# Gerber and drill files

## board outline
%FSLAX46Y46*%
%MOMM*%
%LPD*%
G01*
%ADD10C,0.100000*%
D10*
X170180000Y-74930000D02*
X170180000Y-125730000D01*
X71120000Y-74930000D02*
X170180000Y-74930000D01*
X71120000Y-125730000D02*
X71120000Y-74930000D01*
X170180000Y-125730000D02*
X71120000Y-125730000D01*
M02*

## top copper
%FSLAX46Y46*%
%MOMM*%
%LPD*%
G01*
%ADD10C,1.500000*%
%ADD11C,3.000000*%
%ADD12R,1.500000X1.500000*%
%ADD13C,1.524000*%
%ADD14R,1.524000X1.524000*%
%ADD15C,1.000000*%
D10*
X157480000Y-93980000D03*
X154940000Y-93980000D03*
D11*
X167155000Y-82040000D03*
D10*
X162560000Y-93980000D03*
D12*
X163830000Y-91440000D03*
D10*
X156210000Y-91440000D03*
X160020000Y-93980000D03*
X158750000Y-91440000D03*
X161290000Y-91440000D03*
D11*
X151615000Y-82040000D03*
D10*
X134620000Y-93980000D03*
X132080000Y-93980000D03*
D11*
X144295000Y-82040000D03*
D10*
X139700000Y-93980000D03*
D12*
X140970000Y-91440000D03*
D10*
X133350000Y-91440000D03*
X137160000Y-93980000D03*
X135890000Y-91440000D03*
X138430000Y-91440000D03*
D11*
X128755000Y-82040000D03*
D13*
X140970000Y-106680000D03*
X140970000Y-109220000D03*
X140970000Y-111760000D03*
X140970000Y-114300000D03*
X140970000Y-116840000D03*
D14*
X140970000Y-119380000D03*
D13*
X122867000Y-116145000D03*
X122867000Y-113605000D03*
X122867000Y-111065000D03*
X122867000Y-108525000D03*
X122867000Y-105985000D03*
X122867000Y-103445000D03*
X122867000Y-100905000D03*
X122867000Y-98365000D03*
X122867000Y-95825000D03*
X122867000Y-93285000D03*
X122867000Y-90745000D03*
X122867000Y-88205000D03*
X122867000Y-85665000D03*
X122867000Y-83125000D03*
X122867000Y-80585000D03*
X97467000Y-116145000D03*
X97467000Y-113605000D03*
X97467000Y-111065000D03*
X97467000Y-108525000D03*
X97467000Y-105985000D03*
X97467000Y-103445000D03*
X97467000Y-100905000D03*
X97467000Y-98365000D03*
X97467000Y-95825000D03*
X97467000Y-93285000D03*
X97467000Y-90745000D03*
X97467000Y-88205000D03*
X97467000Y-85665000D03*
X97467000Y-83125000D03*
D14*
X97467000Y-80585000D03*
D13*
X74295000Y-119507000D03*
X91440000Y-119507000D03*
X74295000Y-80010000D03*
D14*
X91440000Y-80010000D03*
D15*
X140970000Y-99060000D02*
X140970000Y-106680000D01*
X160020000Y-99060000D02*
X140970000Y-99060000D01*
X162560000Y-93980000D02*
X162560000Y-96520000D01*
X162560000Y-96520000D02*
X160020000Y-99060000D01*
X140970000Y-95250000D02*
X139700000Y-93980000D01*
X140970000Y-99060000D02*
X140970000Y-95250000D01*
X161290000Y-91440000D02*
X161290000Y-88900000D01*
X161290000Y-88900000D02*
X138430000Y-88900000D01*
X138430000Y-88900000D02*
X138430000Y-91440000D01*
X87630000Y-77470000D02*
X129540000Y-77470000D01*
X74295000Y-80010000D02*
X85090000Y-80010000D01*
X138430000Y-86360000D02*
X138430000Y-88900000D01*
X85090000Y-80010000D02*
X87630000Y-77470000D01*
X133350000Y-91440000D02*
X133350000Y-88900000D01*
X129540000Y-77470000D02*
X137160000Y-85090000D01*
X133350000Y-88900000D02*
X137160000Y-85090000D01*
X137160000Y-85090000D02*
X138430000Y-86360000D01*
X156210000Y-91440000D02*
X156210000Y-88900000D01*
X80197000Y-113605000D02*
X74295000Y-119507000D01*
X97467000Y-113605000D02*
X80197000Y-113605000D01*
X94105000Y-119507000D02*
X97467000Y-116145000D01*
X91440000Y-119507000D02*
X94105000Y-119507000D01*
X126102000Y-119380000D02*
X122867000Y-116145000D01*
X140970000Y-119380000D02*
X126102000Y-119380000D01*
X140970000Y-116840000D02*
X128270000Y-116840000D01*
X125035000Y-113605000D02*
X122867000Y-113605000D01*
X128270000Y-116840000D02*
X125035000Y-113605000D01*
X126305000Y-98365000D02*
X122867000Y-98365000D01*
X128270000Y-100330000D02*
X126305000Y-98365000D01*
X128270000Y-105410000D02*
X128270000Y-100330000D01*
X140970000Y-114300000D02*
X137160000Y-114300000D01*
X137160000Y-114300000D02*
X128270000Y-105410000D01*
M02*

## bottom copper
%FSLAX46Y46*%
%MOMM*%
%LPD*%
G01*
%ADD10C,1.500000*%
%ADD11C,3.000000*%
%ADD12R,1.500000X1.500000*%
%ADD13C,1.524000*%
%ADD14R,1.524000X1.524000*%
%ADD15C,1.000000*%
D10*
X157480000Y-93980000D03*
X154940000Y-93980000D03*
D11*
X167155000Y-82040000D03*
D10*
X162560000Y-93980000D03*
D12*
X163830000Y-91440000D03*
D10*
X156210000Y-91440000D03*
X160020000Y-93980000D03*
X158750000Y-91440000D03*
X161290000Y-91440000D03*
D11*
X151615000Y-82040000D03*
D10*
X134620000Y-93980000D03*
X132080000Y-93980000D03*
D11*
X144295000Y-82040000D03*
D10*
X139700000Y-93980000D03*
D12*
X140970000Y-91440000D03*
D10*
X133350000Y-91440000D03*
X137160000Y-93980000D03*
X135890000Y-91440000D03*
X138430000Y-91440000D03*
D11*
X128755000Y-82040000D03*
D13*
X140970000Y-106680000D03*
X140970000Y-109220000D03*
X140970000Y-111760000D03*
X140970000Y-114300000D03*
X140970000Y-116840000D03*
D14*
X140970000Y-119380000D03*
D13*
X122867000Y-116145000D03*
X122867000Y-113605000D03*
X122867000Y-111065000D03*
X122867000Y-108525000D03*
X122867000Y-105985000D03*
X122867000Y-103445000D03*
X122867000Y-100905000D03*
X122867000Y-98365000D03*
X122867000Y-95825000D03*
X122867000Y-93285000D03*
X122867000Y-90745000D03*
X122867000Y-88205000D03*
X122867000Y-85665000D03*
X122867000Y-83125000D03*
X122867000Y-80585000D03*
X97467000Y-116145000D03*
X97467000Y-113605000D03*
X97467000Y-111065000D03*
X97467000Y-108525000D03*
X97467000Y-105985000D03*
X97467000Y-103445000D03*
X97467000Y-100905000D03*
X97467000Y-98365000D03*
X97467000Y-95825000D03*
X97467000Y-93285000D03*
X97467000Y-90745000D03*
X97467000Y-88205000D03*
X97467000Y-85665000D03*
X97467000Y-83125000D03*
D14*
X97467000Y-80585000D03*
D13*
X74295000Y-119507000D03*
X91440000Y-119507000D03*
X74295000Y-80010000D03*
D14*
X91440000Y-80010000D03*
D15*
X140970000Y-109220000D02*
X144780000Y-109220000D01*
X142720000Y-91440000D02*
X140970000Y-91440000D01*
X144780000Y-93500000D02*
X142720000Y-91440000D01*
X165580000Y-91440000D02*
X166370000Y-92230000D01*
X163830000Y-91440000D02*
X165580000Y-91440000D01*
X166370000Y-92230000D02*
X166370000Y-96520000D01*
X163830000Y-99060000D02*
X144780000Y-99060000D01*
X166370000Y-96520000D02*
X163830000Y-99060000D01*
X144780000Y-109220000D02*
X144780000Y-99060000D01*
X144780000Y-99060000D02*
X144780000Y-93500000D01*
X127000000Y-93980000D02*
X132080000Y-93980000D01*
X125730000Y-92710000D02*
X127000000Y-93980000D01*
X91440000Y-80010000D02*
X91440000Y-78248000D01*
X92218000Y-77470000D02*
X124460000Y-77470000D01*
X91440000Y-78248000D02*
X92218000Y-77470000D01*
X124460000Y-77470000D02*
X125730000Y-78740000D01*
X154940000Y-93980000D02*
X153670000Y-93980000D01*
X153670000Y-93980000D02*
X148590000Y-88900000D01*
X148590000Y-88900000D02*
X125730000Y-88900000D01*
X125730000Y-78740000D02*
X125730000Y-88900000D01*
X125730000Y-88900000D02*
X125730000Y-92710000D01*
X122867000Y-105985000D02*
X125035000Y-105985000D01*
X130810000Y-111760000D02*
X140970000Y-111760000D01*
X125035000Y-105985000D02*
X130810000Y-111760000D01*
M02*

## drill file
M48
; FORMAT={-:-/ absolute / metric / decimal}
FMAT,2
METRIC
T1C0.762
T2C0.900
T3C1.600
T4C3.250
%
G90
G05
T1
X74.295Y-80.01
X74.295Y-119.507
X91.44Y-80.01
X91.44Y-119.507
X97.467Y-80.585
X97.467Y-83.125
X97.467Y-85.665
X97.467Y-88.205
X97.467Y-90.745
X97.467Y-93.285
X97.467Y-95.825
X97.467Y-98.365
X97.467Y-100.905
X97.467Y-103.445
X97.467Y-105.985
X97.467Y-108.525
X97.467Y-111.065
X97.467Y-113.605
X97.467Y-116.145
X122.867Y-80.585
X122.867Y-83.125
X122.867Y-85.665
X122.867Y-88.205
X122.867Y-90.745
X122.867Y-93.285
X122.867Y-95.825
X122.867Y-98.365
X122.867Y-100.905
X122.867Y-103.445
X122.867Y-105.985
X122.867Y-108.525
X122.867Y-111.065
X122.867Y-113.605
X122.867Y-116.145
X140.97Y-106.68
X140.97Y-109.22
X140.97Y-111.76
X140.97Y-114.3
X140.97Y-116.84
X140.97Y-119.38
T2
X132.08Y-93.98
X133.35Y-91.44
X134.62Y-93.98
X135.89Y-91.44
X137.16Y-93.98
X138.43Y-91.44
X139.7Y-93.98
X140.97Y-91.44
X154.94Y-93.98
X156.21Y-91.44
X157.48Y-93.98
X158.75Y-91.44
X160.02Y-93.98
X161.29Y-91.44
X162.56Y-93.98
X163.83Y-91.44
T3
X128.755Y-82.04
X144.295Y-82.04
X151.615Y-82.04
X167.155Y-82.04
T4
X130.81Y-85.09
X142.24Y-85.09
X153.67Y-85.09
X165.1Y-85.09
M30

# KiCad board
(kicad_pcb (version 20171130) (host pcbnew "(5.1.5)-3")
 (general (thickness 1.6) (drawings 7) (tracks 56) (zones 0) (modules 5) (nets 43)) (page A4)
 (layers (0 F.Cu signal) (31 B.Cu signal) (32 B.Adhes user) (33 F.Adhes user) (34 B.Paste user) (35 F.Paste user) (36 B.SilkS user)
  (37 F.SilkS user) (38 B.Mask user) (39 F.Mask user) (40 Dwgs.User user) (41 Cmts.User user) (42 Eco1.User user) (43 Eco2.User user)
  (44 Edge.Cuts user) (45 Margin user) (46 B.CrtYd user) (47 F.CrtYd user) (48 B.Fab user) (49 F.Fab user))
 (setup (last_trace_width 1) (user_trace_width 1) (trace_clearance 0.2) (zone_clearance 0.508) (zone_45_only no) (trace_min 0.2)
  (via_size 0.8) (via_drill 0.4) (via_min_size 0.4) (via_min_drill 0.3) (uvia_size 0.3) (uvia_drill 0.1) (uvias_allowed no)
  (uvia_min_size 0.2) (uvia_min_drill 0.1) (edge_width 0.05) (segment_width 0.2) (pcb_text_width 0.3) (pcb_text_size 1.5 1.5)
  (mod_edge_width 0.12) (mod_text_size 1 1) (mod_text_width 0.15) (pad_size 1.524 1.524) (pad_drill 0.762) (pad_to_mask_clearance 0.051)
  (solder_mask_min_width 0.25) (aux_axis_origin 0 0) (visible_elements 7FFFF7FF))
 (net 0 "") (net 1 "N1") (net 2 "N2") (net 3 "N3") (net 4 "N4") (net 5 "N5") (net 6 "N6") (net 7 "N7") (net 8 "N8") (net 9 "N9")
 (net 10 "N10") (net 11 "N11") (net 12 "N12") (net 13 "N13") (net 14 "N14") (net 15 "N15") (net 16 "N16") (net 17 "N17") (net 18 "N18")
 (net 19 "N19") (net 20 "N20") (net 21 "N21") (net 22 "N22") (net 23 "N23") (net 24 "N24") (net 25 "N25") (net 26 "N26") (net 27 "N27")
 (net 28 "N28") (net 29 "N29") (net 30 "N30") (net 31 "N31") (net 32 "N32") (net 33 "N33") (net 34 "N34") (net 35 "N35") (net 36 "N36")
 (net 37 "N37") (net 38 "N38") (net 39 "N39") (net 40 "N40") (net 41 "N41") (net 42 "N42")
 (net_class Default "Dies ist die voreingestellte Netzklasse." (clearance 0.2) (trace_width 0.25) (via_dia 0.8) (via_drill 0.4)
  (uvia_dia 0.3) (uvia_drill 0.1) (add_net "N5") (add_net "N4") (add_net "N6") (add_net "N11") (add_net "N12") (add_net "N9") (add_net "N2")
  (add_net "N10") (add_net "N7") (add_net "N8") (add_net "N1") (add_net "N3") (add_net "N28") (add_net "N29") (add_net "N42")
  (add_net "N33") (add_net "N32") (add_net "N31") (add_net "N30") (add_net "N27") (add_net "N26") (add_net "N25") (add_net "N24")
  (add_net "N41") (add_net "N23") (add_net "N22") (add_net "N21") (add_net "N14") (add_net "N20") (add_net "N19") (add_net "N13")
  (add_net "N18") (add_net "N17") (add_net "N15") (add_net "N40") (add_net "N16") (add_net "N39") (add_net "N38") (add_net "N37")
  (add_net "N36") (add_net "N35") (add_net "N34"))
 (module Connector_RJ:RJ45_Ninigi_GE (layer F.Cu) (at 163.83 91.44 180)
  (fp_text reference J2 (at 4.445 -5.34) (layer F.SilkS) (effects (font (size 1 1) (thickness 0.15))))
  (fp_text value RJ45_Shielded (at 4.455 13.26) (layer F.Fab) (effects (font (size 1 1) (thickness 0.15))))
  (pad 6 thru_hole circle (at 6.35 -2.54) (size 1.5 1.5) (drill 0.9) (layers *.Cu *.Mask) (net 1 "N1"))
  (pad 8 thru_hole circle (at 8.89 -2.54) (size 1.5 1.5) (drill 0.9) (layers *.Cu *.Mask) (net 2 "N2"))
  (pad SH thru_hole circle (at -3.325 9.4 180) (size 3 3) (drill 1.6) (layers *.Cu *.Mask) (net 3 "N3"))
  (pad 2 thru_hole circle (at 1.27 -2.54) (size 1.5 1.5) (drill 0.9) (layers *.Cu *.Mask) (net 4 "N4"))
  (pad 1 thru_hole rect (at 0 0) (size 1.5 1.5) (drill 0.9) (layers *.Cu *.Mask) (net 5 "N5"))
  (pad 7 thru_hole circle (at 7.62 0) (size 1.5 1.5) (drill 0.9) (layers *.Cu *.Mask) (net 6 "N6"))
  (pad 4 thru_hole circle (at 3.81 -2.54) (size 1.5 1.5) (drill 0.9) (layers *.Cu *.Mask) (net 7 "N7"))
  (pad 5 thru_hole circle (at 5.08 0) (size 1.5 1.5) (drill 0.9) (layers *.Cu *.Mask) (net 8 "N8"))
  (pad 3 thru_hole circle (at 2.54 0) (size 1.5 1.5) (drill 0.9) (layers *.Cu *.Mask) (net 6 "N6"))
  (pad "" np_thru_hole circle (at -1.27 6.35 180) (size 3.25 3.25) (drill 3.25) (layers *.Cu *.Mask))
  (pad SH thru_hole circle (at 12.215 9.4) (size 3 3) (drill 1.6) (layers *.Cu *.Mask) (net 3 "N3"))
  (pad "" np_thru_hole circle (at 10.16 6.35) (size 3.25 3.25) (drill 3.25) (layers *.Cu *.Mask)))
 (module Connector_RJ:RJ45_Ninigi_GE (layer F.Cu) (at 140.97 91.44 180)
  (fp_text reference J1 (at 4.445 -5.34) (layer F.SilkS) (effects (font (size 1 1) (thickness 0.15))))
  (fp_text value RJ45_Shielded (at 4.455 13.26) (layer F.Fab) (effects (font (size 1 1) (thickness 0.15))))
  (pad 6 thru_hole circle (at 6.35 -2.54) (size 1.5 1.5) (drill 0.9) (layers *.Cu *.Mask) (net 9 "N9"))
  (pad 8 thru_hole circle (at 8.89 -2.54) (size 1.5 1.5) (drill 0.9) (layers *.Cu *.Mask) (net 2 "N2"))
  (pad SH thru_hole circle (at -3.325 9.4 180) (size 3 3) (drill 1.6) (layers *.Cu *.Mask) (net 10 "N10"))
  (pad 2 thru_hole circle (at 1.27 -2.54) (size 1.5 1.5) (drill 0.9) (layers *.Cu *.Mask) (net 4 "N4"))
  (pad 1 thru_hole rect (at 0 0) (size 1.5 1.5) (drill 0.9) (layers *.Cu *.Mask) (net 5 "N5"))
  (pad 7 thru_hole circle (at 7.62 0) (size 1.5 1.5) (drill 0.9) (layers *.Cu *.Mask) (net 6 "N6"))
  (pad 4 thru_hole circle (at 3.81 -2.54) (size 1.5 1.5) (drill 0.9) (layers *.Cu *.Mask) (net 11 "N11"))
  (pad 5 thru_hole circle (at 5.08 0) (size 1.5 1.5) (drill 0.9) (layers *.Cu *.Mask) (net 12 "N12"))
  (pad 3 thru_hole circle (at 2.54 0) (size 1.5 1.5) (drill 0.9) (layers *.Cu *.Mask) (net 6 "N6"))
  (pad "" np_thru_hole circle (at -1.27 6.35 180) (size 3.25 3.25) (drill 3.25) (layers *.Cu *.Mask))
  (pad SH thru_hole circle (at 12.215 9.4) (size 3 3) (drill 1.6) (layers *.Cu *.Mask) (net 10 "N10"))
  (pad "" np_thru_hole circle (at 10.16 6.35) (size 3.25 3.25) (drill 3.25) (layers *.Cu *.Mask)))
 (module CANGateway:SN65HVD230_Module (layer F.Cu) (at 140.97 121.92 180)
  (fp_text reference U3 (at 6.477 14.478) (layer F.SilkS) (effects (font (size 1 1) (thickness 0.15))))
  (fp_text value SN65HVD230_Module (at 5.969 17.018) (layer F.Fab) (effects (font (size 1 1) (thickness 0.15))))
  (pad 6 thru_hole circle (at 0 15.24 180) (size 1.524 1.524) (drill 0.762) (layers *.Cu *.Mask) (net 4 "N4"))
  (pad 5 thru_hole circle (at 0 12.7 180) (size 1.524 1.524) (drill 0.762) (layers *.Cu *.Mask) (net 5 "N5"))
  (pad 4 thru_hole circle (at 0 10.16 180) (size 1.524 1.524) (drill 0.762) (layers *.Cu *.Mask) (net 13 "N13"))
  (pad 3 thru_hole circle (at 0 7.62 180) (size 1.524 1.524) (drill 0.762) (layers *.Cu *.Mask) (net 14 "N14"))
  (pad 2 thru_hole circle (at 0 5.08 180) (size 1.524 1.524) (drill 0.762) (layers *.Cu *.Mask) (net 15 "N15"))
  (pad 1 thru_hole rect (at 0 2.54 180) (size 1.524 1.524) (drill 0.762) (layers *.Cu *.Mask) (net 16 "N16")))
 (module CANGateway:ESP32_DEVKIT (layer F.Cu) (at 110.167 95.825)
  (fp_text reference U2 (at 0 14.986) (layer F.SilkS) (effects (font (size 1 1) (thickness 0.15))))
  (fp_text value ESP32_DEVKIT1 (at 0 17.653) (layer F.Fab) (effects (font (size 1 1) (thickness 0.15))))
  (pad 30 thru_hole circle (at 12.7 20.32) (size 1.524 1.524) (drill 0.762) (layers *.Cu *.Mask) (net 16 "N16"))
  (pad 29 thru_hole circle (at 12.7 17.78) (size 1.524 1.524) (drill 0.762) (layers *.Cu *.Mask) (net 15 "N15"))
  (pad 28 thru_hole circle (at 12.7 15.24) (size 1.524 1.524) (drill 0.762) (layers *.Cu *.Mask) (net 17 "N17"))
  (pad 27 thru_hole circle (at 12.7 12.7) (size 1.524 1.524) (drill 0.762) (layers *.Cu *.Mask) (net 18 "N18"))
  (pad 26 thru_hole circle (at 12.7 10.16) (size 1.524 1.524) (drill 0.762) (layers *.Cu *.Mask) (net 13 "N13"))
  (pad 25 thru_hole circle (at 12.7 7.62) (size 1.524 1.524) (drill 0.762) (layers *.Cu *.Mask) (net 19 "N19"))
  (pad 24 thru_hole circle (at 12.7 5.08) (size 1.524 1.524) (drill 0.762) (layers *.Cu *.Mask) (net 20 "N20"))
  (pad 23 thru_hole circle (at 12.7 2.54) (size 1.524 1.524) (drill 0.762) (layers *.Cu *.Mask) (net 14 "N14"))
  (pad 22 thru_hole circle (at 12.7 0) (size 1.524 1.524) (drill 0.762) (layers *.Cu *.Mask) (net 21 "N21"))
  (pad 21 thru_hole circle (at 12.7 -2.54) (size 1.524 1.524) (drill 0.762) (layers *.Cu *.Mask) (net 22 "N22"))
  (pad 20 thru_hole circle (at 12.7 -5.08) (size 1.524 1.524) (drill 0.762) (layers *.Cu *.Mask) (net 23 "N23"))
  (pad 19 thru_hole circle (at 12.7 -7.62) (size 1.524 1.524) (drill 0.762) (layers *.Cu *.Mask) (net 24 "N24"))
  (pad 18 thru_hole circle (at 12.7 -10.16) (size 1.524 1.524) (drill 0.762) (layers *.Cu *.Mask) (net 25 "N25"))
  (pad 17 thru_hole circle (at 12.7 -12.7) (size 1.524 1.524) (drill 0.762) (layers *.Cu *.Mask) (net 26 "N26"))
  (pad 16 thru_hole circle (at 12.7 -15.24) (size 1.524 1.524) (drill 0.762) (layers *.Cu *.Mask) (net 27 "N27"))
  (pad 15 thru_hole circle (at -12.7 20.32) (size 1.524 1.524) (drill 0.762) (layers *.Cu *.Mask) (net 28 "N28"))
  (pad 14 thru_hole circle (at -12.7 17.78) (size 1.524 1.524) (drill 0.762) (layers *.Cu *.Mask) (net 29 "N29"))
  (pad 13 thru_hole circle (at -12.7 15.24) (size 1.524 1.524) (drill 0.762) (layers *.Cu *.Mask) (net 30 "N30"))
  (pad 12 thru_hole circle (at -12.7 12.7) (size 1.524 1.524) (drill 0.762) (layers *.Cu *.Mask) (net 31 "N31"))
  (pad 11 thru_hole circle (at -12.7 10.16) (size 1.524 1.524) (drill 0.762) (layers *.Cu *.Mask) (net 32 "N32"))
  (pad 10 thru_hole circle (at -12.7 7.62) (size 1.524 1.524) (drill 0.762) (layers *.Cu *.Mask) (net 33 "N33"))
  (pad 9 thru_hole circle (at -12.7 5.08) (size 1.524 1.524) (drill 0.762) (layers *.Cu *.Mask) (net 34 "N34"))
  (pad 8 thru_hole circle (at -12.7 2.54) (size 1.524 1.524) (drill 0.762) (layers *.Cu *.Mask) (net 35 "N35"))
  (pad 7 thru_hole circle (at -12.7 0) (size 1.524 1.524) (drill 0.762) (layers *.Cu *.Mask) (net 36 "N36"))
  (pad 6 thru_hole circle (at -12.7 -2.54) (size 1.524 1.524) (drill 0.762) (layers *.Cu *.Mask) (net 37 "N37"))
  (pad 5 thru_hole circle (at -12.7 -5.08) (size 1.524 1.524) (drill 0.762) (layers *.Cu *.Mask) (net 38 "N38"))
  (pad 4 thru_hole circle (at -12.7 -7.62) (size 1.524 1.524) (drill 0.762) (layers *.Cu *.Mask) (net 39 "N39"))
  (pad 3 thru_hole circle (at -12.7 -10.16) (size 1.524 1.524) (drill 0.762) (layers *.Cu *.Mask) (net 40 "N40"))
  (pad 2 thru_hole circle (at -12.7 -12.7) (size 1.524 1.524) (drill 0.762) (layers *.Cu *.Mask) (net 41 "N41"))
  (pad 1 thru_hole rect (at -12.7 -15.24) (size 1.524 1.524) (drill 0.762) (layers *.Cu *.Mask) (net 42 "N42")))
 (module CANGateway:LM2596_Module (layer F.Cu) (at 82.55 100.33 270)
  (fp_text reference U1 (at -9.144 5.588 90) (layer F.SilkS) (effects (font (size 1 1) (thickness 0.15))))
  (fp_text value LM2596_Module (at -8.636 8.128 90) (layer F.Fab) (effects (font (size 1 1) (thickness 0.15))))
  (pad 4 thru_hole circle (at 19.177 8.255 270) (size 1.524 1.524) (drill 0.762) (layers *.Cu *.Mask) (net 29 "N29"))
  (pad 3 thru_hole circle (at 19.177 -8.89 270) (size 1.524 1.524) (drill 0.762) (layers *.Cu *.Mask) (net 28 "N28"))
  (pad 2 thru_hole circle (at -20.32 8.255 270) (size 1.524 1.524) (drill 0.762) (layers *.Cu *.Mask) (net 6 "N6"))
  (pad 1 thru_hole rect (at -20.32 -8.89 270) (size 1.524 1.524) (drill 0.762) (layers *.Cu *.Mask) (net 2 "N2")))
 (gr_line (start 170.18 74.93) (end 170.18 125.73) (layer Edge.Cuts) (width 0.1))
 (gr_line (start 71.12 74.93) (end 170.18 74.93) (layer Edge.Cuts) (width 0.1))
 (gr_line (start 71.12 125.73) (end 71.12 74.93) (layer Edge.Cuts) (width 0.1))
 (gr_line (start 170.18 125.73) (end 71.12 125.73) (layer Edge.Cuts) (width 0.1))
 (segment (start 140.97 109.22) (end 144.78 109.22) (width 1) (layer B.Cu) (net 5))
 (segment (start 142.72 91.44) (end 140.97 91.44) (width 1) (layer B.Cu) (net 5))
 (segment (start 144.78 93.5) (end 142.72 91.44) (width 1) (layer B.Cu) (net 5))
 (segment (start 165.58 91.44) (end 166.37 92.23) (width 1) (layer B.Cu) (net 5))
 (segment (start 163.83 91.44) (end 165.58 91.44) (width 1) (layer B.Cu) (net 5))
 (segment (start 166.37 92.23) (end 166.37 96.52) (width 1) (layer B.Cu) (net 5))
 (segment (start 163.83 99.06) (end 144.78 99.06) (width 1) (layer B.Cu) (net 5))
 (segment (start 166.37 96.52) (end 163.83 99.06) (width 1) (layer B.Cu) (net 5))
 (segment (start 144.78 109.22) (end 144.78 99.06) (width 1) (layer B.Cu) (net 5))
 (segment (start 144.78 99.06) (end 144.78 93.5) (width 1) (layer B.Cu) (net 5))
 (segment (start 140.97 99.06) (end 140.97 106.68) (width 1) (layer F.Cu) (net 4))
 (segment (start 160.02 99.06) (end 140.97 99.06) (width 1) (layer F.Cu) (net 4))
 (segment (start 162.56 93.98) (end 162.56 96.52) (width 1) (layer F.Cu) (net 4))
 (segment (start 162.56 96.52) (end 160.02 99.06) (width 1) (layer F.Cu) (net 4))
 (segment (start 140.97 95.25) (end 139.7 93.98) (width 1) (layer F.Cu) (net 4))
 (segment (start 140.97 99.06) (end 140.97 95.25) (width 1) (layer F.Cu) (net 4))
 (segment (start 161.29 91.44) (end 161.29 88.9) (width 1) (layer F.Cu) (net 6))
 (segment (start 161.29 88.9) (end 138.43 88.9) (width 1) (layer F.Cu) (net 6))
 (segment (start 138.43 88.9) (end 138.43 91.44) (width 1) (layer F.Cu) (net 6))
 (segment (start 87.63 77.47) (end 129.54 77.47) (width 1) (layer F.Cu) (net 6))
 (segment (start 74.295 80.01) (end 85.09 80.01) (width 1) (layer F.Cu) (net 6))
 (segment (start 138.43 86.36) (end 138.43 88.9) (width 1) (layer F.Cu) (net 6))
 (segment (start 85.09 80.01) (end 87.63 77.47) (width 1) (layer F.Cu) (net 6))
 (segment (start 133.35 91.44) (end 133.35 88.9) (width 1) (layer F.Cu) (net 6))
 (segment (start 129.54 77.47) (end 137.16 85.09) (width 1) (layer F.Cu) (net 6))
 (segment (start 133.35 88.9) (end 137.16 85.09) (width 1) (layer F.Cu) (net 6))
 (segment (start 137.16 85.09) (end 138.43 86.36) (width 1) (layer F.Cu) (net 6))
 (segment (start 156.21 91.44) (end 156.21 88.9) (width 1) (layer F.Cu) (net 6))
 (segment (start 127 93.98) (end 132.08 93.98) (width 1) (layer B.Cu) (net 2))
 (segment (start 125.73 92.71) (end 127 93.98) (width 1) (layer B.Cu) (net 2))
 (segment (start 91.44 80.01) (end 91.44 78.248) (width 1) (layer B.Cu) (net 2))
 (segment (start 92.218 77.47) (end 124.46 77.47) (width 1) (layer B.Cu) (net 2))
 (segment (start 91.44 78.248) (end 92.218 77.47) (width 1) (layer B.Cu) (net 2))
 (segment (start 124.46 77.47) (end 125.73 78.74) (width 1) (layer B.Cu) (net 2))
 (segment (start 154.94 93.98) (end 153.67 93.98) (width 1) (layer B.Cu) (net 2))
 (segment (start 153.67 93.98) (end 148.59 88.9) (width 1) (layer B.Cu) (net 2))
 (segment (start 148.59 88.9) (end 125.73 88.9) (width 1) (layer B.Cu) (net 2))
 (segment (start 125.73 78.74) (end 125.73 88.9) (width 1) (layer B.Cu) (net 2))
 (segment (start 125.73 88.9) (end 125.73 92.71) (width 1) (layer B.Cu) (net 2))
 (segment (start 80.197 113.605) (end 74.295 119.507) (width 1) (layer F.Cu) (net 29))
 (segment (start 97.467 113.605) (end 80.197 113.605) (width 1) (layer F.Cu) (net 29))
 (segment (start 94.105 119.507) (end 97.467 116.145) (width 1) (layer F.Cu) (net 28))
 (segment (start 91.44 119.507) (end 94.105 119.507) (width 1) (layer F.Cu) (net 28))
 (segment (start 126.102 119.38) (end 122.867 116.145) (width 1) (layer F.Cu) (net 16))
 (segment (start 140.97 119.38) (end 126.102 119.38) (width 1) (layer F.Cu) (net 16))
 (segment (start 140.97 116.84) (end 128.27 116.84) (width 1) (layer F.Cu) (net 15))
 (segment (start 125.035 113.605) (end 122.867 113.605) (width 1) (layer F.Cu) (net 15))
 (segment (start 128.27 116.84) (end 125.035 113.605) (width 1) (layer F.Cu) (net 15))
 (segment (start 122.867 105.985) (end 125.035 105.985) (width 1) (layer B.Cu) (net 13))
 (segment (start 130.81 111.76) (end 140.97 111.76) (width 1) (layer B.Cu) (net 13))
 (segment (start 125.035 105.985) (end 130.81 111.76) (width 1) (layer B.Cu) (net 13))
 (segment (start 126.305 98.365) (end 122.867 98.365) (width 1) (layer F.Cu) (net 14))
 (segment (start 128.27 100.33) (end 126.305 98.365) (width 1) (layer F.Cu) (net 14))
 (segment (start 128.27 105.41) (end 128.27 100.33) (width 1) (layer F.Cu) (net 14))
 (segment (start 140.97 114.3) (end 137.16 114.3) (width 1) (layer F.Cu) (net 14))
 (segment (start 137.16 114.3) (end 128.27 105.41) (width 1) (layer F.Cu) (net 14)))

